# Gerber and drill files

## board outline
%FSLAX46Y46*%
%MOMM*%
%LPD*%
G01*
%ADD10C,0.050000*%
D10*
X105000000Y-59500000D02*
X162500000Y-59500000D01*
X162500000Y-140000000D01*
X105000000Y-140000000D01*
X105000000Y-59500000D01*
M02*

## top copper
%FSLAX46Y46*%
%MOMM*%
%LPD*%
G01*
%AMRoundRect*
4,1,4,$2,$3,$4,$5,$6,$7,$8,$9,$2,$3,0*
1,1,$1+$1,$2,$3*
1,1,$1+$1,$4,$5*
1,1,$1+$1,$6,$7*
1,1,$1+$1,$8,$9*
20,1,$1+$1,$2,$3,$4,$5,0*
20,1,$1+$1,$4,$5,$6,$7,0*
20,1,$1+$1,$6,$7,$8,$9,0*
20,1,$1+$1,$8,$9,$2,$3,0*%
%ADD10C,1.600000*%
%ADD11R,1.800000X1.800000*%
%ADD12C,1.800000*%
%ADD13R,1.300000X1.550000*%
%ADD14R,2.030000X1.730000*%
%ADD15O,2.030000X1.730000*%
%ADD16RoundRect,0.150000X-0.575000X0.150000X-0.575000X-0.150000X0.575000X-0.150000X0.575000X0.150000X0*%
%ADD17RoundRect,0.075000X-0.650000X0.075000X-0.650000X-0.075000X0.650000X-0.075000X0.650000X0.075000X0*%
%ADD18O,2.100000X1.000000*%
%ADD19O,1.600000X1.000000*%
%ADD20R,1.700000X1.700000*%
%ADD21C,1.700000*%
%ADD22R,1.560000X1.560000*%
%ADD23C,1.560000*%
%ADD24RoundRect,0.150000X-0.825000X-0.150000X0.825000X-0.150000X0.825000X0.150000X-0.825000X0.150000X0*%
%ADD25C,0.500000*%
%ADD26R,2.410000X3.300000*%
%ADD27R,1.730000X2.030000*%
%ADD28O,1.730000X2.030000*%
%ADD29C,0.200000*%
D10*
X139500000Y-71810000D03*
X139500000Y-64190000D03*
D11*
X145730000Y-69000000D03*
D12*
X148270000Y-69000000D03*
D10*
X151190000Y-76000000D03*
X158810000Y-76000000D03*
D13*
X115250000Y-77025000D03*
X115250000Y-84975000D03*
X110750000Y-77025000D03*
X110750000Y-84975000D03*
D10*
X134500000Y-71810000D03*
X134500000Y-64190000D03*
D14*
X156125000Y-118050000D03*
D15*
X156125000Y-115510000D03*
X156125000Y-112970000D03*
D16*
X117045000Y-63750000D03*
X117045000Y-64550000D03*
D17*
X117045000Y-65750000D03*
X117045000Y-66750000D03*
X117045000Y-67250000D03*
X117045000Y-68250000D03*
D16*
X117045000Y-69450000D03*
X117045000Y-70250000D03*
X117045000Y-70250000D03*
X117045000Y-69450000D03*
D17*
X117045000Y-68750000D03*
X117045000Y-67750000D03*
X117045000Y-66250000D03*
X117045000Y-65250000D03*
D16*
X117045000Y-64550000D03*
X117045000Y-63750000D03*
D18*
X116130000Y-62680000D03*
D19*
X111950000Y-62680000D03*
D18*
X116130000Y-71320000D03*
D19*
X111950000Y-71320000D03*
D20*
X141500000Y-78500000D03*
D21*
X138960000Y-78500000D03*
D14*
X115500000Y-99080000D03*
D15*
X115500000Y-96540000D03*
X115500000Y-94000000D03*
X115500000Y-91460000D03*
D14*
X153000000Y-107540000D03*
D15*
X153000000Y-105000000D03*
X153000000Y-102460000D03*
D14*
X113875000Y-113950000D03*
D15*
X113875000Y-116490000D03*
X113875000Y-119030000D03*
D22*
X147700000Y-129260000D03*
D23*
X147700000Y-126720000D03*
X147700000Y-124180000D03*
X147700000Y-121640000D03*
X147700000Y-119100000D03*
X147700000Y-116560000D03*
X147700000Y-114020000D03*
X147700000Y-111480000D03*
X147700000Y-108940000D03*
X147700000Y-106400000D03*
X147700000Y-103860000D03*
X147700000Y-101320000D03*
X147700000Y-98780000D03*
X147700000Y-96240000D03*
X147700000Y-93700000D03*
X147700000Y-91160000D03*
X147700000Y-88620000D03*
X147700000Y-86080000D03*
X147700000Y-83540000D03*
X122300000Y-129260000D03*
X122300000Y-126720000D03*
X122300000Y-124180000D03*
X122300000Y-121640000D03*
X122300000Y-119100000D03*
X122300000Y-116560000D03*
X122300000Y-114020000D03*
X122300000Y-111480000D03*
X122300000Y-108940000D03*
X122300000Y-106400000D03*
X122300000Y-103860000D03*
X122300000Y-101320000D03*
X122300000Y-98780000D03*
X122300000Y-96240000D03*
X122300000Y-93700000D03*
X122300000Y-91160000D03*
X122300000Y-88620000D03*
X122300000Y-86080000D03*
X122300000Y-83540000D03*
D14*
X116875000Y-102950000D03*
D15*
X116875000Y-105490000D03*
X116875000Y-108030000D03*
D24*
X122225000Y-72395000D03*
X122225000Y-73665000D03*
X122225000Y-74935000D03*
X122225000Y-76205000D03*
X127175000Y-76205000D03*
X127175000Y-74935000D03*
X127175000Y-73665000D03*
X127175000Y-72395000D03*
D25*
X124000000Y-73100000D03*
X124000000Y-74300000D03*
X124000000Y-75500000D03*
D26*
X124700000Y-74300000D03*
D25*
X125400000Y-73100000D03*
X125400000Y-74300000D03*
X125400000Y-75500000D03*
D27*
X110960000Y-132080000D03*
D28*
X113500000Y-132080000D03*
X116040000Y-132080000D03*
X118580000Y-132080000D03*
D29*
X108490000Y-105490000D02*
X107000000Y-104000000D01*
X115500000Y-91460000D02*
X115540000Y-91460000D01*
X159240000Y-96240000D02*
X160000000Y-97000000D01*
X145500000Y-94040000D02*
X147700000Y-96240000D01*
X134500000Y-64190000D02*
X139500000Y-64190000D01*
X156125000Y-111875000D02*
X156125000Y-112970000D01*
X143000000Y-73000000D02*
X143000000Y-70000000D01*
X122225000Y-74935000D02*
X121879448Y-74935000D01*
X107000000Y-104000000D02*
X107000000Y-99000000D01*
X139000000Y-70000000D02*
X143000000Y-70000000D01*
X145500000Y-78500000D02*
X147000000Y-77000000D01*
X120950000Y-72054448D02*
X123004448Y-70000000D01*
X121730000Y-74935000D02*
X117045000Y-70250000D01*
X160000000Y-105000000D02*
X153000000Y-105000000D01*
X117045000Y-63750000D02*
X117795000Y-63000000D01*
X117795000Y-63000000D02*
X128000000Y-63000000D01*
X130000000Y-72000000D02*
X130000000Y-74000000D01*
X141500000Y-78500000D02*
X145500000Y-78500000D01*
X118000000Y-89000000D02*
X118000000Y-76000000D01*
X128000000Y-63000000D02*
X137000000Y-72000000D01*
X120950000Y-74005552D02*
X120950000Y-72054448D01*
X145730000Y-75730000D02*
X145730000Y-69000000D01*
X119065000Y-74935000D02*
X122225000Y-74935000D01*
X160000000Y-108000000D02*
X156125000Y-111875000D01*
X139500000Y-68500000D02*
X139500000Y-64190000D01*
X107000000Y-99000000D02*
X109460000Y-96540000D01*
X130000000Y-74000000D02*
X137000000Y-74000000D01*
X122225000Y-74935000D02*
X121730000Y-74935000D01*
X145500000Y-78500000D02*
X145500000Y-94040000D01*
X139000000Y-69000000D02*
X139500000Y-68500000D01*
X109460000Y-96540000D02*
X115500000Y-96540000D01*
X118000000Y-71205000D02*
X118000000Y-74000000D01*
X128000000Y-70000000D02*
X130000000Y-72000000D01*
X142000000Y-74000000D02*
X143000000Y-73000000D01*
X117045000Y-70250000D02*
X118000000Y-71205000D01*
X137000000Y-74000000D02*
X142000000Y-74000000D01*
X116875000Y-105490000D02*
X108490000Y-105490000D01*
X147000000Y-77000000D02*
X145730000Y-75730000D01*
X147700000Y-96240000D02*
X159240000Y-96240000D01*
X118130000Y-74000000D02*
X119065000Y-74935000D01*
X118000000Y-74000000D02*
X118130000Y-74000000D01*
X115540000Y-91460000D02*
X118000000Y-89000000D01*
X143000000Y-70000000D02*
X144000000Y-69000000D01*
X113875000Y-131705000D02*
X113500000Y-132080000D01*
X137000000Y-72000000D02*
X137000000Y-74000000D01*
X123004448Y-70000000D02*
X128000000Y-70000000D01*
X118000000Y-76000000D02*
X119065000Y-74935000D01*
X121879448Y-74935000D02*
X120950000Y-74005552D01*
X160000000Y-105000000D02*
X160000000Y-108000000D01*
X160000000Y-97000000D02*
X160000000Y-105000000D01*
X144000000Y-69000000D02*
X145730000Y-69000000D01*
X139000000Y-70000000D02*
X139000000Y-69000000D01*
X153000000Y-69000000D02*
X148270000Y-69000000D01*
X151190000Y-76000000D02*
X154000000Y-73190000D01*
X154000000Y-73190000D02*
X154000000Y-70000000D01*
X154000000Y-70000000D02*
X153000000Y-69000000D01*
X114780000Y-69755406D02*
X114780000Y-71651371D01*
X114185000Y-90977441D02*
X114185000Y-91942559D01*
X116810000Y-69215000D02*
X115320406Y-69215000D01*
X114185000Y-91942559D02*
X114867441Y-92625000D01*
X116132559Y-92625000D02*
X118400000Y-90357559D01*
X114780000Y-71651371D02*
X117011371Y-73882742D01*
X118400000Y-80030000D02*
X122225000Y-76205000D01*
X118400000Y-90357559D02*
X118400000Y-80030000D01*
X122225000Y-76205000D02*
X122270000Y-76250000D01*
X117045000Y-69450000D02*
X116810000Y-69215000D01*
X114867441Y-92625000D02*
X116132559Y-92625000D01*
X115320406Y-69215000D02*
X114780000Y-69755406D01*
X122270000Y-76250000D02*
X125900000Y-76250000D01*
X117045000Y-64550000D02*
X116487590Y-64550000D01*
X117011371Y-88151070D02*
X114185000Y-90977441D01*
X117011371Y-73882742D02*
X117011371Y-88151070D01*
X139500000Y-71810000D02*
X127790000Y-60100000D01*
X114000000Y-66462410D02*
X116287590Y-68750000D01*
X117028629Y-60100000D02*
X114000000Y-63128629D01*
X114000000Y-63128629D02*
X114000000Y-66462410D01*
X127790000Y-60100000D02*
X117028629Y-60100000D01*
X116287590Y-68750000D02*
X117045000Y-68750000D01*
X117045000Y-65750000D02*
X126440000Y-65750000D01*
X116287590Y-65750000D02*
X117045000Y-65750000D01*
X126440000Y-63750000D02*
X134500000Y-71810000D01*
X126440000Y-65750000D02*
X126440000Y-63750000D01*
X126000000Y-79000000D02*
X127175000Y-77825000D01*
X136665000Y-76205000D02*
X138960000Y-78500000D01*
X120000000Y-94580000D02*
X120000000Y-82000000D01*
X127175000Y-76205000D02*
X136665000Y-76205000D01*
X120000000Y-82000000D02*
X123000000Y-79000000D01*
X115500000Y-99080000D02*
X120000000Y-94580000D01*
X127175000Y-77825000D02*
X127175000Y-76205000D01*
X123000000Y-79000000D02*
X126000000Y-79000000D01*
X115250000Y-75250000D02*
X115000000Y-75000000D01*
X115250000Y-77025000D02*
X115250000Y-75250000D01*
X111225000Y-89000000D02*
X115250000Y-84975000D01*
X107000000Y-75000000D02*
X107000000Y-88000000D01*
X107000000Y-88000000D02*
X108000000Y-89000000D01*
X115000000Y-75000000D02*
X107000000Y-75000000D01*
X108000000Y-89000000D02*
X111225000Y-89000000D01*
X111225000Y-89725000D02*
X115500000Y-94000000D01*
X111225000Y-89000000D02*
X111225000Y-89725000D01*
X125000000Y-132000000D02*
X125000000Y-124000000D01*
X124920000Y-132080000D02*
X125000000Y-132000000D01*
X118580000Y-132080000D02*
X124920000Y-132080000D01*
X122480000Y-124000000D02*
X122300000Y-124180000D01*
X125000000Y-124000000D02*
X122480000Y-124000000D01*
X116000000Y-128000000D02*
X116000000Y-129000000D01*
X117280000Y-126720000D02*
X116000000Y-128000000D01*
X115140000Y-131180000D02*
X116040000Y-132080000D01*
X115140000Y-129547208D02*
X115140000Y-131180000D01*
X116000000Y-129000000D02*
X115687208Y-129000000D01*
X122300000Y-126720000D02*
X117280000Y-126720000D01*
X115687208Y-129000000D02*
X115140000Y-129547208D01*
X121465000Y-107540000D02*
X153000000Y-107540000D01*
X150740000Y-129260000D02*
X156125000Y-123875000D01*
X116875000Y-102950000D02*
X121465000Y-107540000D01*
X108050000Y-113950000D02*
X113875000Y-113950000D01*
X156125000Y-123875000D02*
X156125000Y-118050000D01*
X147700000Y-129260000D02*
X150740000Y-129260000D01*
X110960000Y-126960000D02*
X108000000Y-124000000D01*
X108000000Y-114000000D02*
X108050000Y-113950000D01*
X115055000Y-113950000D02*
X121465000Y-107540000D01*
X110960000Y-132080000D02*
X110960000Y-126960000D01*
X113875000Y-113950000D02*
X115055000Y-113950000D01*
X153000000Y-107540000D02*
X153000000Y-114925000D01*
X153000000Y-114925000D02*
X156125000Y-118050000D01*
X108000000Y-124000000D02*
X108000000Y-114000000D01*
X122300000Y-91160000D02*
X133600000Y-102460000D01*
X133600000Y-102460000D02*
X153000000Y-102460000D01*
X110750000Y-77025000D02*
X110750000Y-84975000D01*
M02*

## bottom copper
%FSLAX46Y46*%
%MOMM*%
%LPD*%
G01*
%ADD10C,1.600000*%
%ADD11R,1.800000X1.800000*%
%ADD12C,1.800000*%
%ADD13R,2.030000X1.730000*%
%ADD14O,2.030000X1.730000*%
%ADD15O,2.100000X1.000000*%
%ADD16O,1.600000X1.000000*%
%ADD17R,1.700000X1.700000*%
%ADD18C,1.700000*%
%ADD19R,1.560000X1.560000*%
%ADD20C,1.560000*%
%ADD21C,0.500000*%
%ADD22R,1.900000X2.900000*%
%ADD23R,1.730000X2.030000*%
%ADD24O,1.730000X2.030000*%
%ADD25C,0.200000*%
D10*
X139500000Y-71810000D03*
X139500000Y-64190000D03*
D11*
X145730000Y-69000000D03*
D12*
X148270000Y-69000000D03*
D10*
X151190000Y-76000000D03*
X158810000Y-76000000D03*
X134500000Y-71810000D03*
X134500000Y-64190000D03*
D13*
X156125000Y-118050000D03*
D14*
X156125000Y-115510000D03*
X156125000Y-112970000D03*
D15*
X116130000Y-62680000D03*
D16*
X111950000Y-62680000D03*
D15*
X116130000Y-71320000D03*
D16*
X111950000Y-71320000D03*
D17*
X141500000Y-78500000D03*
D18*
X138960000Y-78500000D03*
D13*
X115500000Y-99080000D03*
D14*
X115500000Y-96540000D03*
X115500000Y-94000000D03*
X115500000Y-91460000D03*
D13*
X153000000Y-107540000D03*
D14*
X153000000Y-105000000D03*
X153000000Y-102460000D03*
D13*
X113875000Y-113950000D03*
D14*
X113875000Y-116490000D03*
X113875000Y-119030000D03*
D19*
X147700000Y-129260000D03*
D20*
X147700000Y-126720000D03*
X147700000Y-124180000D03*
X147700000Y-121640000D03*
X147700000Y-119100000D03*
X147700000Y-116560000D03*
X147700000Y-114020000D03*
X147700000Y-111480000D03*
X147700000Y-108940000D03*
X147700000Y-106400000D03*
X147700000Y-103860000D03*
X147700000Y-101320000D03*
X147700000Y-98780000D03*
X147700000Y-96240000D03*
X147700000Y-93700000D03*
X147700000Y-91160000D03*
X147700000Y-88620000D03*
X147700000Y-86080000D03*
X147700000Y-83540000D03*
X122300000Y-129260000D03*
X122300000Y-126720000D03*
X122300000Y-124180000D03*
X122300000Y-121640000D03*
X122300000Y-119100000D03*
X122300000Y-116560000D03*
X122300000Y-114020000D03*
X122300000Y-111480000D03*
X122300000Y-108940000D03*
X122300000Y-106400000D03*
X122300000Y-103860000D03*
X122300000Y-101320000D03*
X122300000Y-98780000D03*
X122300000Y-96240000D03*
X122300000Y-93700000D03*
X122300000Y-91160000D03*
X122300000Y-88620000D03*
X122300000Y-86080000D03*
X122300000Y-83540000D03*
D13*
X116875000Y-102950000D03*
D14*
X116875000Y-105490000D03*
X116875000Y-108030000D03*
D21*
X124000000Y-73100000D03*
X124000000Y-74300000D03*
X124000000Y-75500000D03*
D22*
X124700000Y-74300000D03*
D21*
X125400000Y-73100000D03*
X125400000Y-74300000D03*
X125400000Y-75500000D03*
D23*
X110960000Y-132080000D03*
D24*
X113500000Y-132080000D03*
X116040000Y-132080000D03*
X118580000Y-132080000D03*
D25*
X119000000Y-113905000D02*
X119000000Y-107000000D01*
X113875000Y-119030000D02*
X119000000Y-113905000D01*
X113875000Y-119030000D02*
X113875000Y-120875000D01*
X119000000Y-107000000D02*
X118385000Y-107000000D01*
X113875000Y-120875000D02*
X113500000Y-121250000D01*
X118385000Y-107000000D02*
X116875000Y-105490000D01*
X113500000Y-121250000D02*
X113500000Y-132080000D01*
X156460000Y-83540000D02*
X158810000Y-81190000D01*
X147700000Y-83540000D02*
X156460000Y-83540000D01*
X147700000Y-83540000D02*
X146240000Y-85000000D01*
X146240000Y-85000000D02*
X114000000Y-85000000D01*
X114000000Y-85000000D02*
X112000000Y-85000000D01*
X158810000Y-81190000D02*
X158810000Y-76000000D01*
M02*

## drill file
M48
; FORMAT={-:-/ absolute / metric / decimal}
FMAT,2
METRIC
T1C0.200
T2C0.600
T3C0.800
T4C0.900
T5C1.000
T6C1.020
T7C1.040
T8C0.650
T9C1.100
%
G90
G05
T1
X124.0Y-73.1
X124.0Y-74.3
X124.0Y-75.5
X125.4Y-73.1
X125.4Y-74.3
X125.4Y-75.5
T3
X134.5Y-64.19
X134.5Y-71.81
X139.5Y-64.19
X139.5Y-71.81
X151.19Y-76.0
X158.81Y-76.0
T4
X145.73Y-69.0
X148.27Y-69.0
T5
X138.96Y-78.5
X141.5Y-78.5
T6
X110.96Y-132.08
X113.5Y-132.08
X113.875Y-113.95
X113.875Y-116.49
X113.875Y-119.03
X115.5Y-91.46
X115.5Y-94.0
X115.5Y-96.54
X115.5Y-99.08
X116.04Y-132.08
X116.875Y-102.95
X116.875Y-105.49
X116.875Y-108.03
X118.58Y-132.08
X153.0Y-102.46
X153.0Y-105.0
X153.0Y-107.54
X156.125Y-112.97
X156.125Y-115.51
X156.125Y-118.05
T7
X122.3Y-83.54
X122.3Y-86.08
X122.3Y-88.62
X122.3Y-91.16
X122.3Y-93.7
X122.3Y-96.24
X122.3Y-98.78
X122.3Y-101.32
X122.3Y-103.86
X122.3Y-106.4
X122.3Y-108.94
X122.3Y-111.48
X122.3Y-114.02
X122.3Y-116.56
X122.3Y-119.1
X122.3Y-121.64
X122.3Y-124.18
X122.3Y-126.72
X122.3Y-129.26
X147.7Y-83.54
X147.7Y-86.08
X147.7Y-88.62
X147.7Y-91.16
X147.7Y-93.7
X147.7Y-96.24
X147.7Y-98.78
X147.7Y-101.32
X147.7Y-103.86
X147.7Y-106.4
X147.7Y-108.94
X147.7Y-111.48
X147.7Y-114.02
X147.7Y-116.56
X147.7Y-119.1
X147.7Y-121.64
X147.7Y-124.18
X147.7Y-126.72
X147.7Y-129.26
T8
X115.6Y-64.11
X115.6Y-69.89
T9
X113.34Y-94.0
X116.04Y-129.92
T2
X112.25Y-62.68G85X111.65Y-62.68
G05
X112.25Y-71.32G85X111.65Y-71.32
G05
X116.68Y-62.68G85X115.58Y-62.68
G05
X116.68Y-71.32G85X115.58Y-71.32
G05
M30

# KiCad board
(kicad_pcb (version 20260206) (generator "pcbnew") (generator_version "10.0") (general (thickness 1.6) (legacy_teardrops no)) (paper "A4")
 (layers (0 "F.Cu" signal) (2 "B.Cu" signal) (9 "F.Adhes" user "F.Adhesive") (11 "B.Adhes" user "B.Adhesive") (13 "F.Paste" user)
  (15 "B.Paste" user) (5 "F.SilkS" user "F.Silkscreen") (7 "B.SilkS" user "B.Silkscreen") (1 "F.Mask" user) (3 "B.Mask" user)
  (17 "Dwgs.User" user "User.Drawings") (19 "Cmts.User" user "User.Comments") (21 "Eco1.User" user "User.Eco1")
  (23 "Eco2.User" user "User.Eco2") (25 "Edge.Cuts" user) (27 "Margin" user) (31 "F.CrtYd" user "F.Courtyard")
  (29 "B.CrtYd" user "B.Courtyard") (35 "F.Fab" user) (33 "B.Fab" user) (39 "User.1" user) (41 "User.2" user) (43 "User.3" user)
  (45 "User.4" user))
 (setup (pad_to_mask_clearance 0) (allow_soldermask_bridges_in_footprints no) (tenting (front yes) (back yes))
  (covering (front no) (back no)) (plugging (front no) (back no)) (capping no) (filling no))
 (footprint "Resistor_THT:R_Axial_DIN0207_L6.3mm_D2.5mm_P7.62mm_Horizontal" (layer "F.Cu") (at 139.5 71.81 90)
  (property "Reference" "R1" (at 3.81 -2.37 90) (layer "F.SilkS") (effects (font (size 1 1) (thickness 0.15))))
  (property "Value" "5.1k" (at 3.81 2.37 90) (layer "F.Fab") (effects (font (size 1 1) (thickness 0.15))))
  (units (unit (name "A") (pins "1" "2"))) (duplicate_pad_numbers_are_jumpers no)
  (pad "1" thru_hole circle (at 0 0 90) (size 1.6 1.6) (drill 0.8) (layers "*.Cu" "*.Mask") (remove_unused_layers no) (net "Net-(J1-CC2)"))
  (pad "2" thru_hole circle (at 7.62 0 90) (size 1.6 1.6) (drill 0.8) (layers "*.Cu" "*.Mask") (remove_unused_layers no) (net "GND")))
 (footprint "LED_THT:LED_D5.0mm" (layer "F.Cu") (at 145.73 69)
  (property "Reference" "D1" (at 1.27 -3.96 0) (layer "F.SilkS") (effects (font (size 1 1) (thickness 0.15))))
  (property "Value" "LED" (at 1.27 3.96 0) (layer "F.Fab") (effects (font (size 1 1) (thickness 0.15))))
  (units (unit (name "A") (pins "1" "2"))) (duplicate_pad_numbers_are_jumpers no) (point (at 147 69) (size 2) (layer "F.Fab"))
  (pad "1" thru_hole rect (at 0 0) (size 1.8 1.8) (drill 0.9) (layers "*.Cu" "*.Mask") (remove_unused_layers no) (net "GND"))
  (pad "2" thru_hole circle (at 2.54 0) (size 1.8 1.8) (drill 0.9) (layers "*.Cu" "*.Mask") (remove_unused_layers no) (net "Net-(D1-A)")))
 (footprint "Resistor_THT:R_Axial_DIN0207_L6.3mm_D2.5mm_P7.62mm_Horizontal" (layer "F.Cu") (at 151.19 76)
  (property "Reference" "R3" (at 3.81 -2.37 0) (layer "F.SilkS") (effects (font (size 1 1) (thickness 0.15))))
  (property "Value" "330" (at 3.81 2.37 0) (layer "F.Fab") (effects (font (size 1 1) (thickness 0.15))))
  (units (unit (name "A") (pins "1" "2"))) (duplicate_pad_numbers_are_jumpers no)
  (pad "1" thru_hole circle (at 0 0) (size 1.6 1.6) (drill 0.8) (layers "*.Cu" "*.Mask") (remove_unused_layers no) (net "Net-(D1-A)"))
  (pad "2" thru_hole circle (at 7.62 0) (size 1.6 1.6) (drill 0.8) (layers "*.Cu" "*.Mask") (remove_unused_layers no) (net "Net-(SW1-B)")))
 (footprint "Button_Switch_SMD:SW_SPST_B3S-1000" (layer "F.Cu") (at 113 81 -90)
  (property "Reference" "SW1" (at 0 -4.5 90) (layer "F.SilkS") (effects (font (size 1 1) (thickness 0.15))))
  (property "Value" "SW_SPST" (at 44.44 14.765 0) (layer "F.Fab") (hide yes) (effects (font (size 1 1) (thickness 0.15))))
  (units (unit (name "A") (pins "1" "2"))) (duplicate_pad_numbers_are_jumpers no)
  (pad "1" smd rect (at -3.975 -2.25 270) (size 1.55 1.3) (layers "F.Cu" "F.Mask" "F.Paste") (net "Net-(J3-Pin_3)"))
  (pad "1" smd rect (at 3.975 -2.25 270) (size 1.55 1.3) (layers "F.Cu" "F.Mask" "F.Paste") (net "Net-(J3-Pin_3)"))
  (pad "2" smd rect (at -3.975 2.25 270) (size 1.55 1.3) (layers "F.Cu" "F.Mask" "F.Paste") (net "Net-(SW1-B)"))
  (pad "2" smd rect (at 3.975 2.25 270) (size 1.55 1.3) (layers "F.Cu" "F.Mask" "F.Paste") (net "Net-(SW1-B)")))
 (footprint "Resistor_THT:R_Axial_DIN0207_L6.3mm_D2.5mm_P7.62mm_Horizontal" (layer "F.Cu") (at 134.5 71.81 90)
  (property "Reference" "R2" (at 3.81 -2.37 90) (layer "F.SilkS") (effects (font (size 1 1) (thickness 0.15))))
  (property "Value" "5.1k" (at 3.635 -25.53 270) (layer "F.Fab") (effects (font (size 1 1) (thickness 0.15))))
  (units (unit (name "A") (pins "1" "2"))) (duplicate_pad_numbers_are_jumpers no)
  (pad "1" thru_hole circle (at 0 0 90) (size 1.6 1.6) (drill 0.8) (layers "*.Cu" "*.Mask") (remove_unused_layers no) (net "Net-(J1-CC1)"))
  (pad "2" thru_hole circle (at 7.62 0 90) (size 1.6 1.6) (drill 0.8) (layers "*.Cu" "*.Mask") (remove_unused_layers no) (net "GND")))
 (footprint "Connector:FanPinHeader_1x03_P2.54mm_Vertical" (layer "F.Cu") (at 156.125 118.05 90)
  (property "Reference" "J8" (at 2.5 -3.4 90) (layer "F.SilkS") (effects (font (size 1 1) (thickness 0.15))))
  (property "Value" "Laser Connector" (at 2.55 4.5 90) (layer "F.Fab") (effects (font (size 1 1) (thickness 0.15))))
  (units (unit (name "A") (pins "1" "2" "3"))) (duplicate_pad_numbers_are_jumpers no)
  (pad "1" thru_hole rect (at 0 0 180) (size 2.03 1.73) (drill 1.02) (layers "*.Cu" "*.Mask") (remove_unused_layers no)
   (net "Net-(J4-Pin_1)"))
  (pad "2" thru_hole oval (at 2.54 0 180) (size 2.03 1.73) (drill 1.02) (layers "*.Cu" "*.Mask") (remove_unused_layers no)
   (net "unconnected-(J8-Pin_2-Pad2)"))
  (pad "3" thru_hole oval (at 5.08 0 180) (size 2.03 1.73) (drill 1.02) (layers "*.Cu" "*.Mask") (remove_unused_layers no) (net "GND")))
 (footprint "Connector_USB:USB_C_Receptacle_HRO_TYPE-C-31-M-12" (layer "F.Cu") (at 113 67 -90)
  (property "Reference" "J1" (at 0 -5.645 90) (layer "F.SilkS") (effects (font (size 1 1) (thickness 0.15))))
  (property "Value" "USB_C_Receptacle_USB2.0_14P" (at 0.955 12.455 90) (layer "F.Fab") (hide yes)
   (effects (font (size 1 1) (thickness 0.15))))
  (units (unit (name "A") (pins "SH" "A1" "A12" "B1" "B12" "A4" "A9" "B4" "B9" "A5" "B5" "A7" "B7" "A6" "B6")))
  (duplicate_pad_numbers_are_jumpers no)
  (pad "" np_thru_hole circle (at -2.89 -2.6 270) (size 0.65 0.65) (drill 0.65) (layers "*.Cu" "*.Mask"))
  (pad "" np_thru_hole circle (at 2.89 -2.6 270) (size 0.65 0.65) (drill 0.65) (layers "*.Cu" "*.Mask"))
  (pad "A1" smd roundrect (at -3.25 -4.045 270) (size 0.6 1.45) (layers "F.Cu" "F.Mask" "F.Paste") (roundrect_rratio 0.25) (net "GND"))
  (pad "A4" smd roundrect (at -2.45 -4.045 270) (size 0.6 1.45) (layers "F.Cu" "F.Mask" "F.Paste") (roundrect_rratio 0.25)
   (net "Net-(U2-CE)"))
  (pad "A5" smd roundrect (at -1.25 -4.045 270) (size 0.3 1.45) (layers "F.Cu" "F.Mask" "F.Paste") (roundrect_rratio 0.25)
   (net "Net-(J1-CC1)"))
  (pad "A6" smd roundrect (at -0.25 -4.045 270) (size 0.3 1.45) (layers "F.Cu" "F.Mask" "F.Paste") (roundrect_rratio 0.25)
   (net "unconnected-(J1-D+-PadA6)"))
  (pad "A7" smd roundrect (at 0.25 -4.045 270) (size 0.3 1.45) (layers "F.Cu" "F.Mask" "F.Paste") (roundrect_rratio 0.25)
   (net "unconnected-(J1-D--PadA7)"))
  (pad "A8" smd roundrect (at 1.25 -4.045 270) (size 0.3 1.45) (layers "F.Cu" "F.Mask" "F.Paste") (roundrect_rratio 0.25))
  (pad "A9" smd roundrect (at 2.45 -4.045 270) (size 0.6 1.45) (layers "F.Cu" "F.Mask" "F.Paste") (roundrect_rratio 0.25)
   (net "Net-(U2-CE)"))
  (pad "A12" smd roundrect (at 3.25 -4.045 270) (size 0.6 1.45) (layers "F.Cu" "F.Mask" "F.Paste") (roundrect_rratio 0.25) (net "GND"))
  (pad "B1" smd roundrect (at 3.25 -4.045 270) (size 0.6 1.45) (layers "F.Cu" "F.Mask" "F.Paste") (roundrect_rratio 0.25) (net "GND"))
  (pad "B4" smd roundrect (at 2.45 -4.045 270) (size 0.6 1.45) (layers "F.Cu" "F.Mask" "F.Paste") (roundrect_rratio 0.25)
   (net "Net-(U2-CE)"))
  (pad "B5" smd roundrect (at 1.75 -4.045 270) (size 0.3 1.45) (layers "F.Cu" "F.Mask" "F.Paste") (roundrect_rratio 0.25)
   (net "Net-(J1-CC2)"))
  (pad "B6" smd roundrect (at 0.75 -4.045 270) (size 0.3 1.45) (layers "F.Cu" "F.Mask" "F.Paste") (roundrect_rratio 0.25)
   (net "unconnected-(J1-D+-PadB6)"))
  (pad "B7" smd roundrect (at -0.75 -4.045 270) (size 0.3 1.45) (layers "F.Cu" "F.Mask" "F.Paste") (roundrect_rratio 0.25)
   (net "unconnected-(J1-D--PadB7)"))
  (pad "B8" smd roundrect (at -1.75 -4.045 270) (size 0.3 1.45) (layers "F.Cu" "F.Mask" "F.Paste") (roundrect_rratio 0.25))
  (pad "B9" smd roundrect (at -2.45 -4.045 270) (size 0.6 1.45) (layers "F.Cu" "F.Mask" "F.Paste") (roundrect_rratio 0.25)
   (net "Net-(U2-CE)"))
  (pad "B12" smd roundrect (at -3.25 -4.045 270) (size 0.6 1.45) (layers "F.Cu" "F.Mask" "F.Paste") (roundrect_rratio 0.25) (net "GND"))
  (pad "SH" thru_hole oval (at -4.32 -3.13 270) (size 1 2.1) (drill oval 0.6 1.7) (layers "*.Cu" "*.Mask") (remove_unused_layers no)
   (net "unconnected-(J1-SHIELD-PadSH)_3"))
  (pad "SH" thru_hole oval (at -4.32 1.05 270) (size 1 1.6) (drill oval 0.6 1.2) (layers "*.Cu" "*.Mask") (remove_unused_layers no)
   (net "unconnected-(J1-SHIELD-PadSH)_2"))
  (pad "SH" thru_hole oval (at 4.32 -3.13 270) (size 1 2.1) (drill oval 0.6 1.7) (layers "*.Cu" "*.Mask") (remove_unused_layers no)
   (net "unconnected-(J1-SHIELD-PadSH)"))
  (pad "SH" thru_hole oval (at 4.32 1.05 270) (size 1 1.6) (drill oval 0.6 1.2) (layers "*.Cu" "*.Mask") (remove_unused_layers no)
   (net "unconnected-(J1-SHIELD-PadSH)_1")))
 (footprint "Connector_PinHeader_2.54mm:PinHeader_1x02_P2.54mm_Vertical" (layer "F.Cu") (at 141.5 78.5 -90)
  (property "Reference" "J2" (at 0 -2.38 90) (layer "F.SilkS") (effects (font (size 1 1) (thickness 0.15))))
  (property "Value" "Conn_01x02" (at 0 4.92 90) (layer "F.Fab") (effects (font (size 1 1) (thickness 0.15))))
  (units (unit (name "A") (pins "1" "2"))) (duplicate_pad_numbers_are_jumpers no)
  (pad "1" thru_hole rect (at 0 0 270) (size 1.7 1.7) (drill 1) (layers "*.Cu" "*.Mask") (remove_unused_layers no) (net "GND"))
  (pad "2" thru_hole circle (at 0 2.54 270) (size 1.7 1.7) (drill 1) (layers "*.Cu" "*.Mask") (remove_unused_layers no)
   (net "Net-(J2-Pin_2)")))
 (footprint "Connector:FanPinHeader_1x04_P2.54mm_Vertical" (layer "F.Cu") (at 115.5 99.08 90)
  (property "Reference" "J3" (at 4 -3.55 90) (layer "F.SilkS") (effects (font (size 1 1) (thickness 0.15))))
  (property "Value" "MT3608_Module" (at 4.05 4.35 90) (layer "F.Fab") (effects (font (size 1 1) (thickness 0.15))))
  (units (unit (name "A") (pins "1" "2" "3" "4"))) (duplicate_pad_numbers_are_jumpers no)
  (pad "" np_thru_hole circle (at 5.08 -2.16 180) (size 1.1 1.1) (drill 1.1) (layers "*.Cu" "*.Mask"))
  (pad "1" thru_hole rect (at 0 0 180) (size 2.03 1.73) (drill 1.02) (layers "*.Cu" "*.Mask") (remove_unused_layers no)
   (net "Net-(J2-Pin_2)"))
  (pad "2" thru_hole oval (at 2.54 0 180) (size 2.03 1.73) (drill 1.02) (layers "*.Cu" "*.Mask") (remove_unused_layers no) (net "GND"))
  (pad "3" thru_hole oval (at 5.08 0 180) (size 2.03 1.73) (drill 1.02) (layers "*.Cu" "*.Mask") (remove_unused_layers no)
   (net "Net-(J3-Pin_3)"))
  (pad "4" thru_hole oval (at 7.62 0 180) (size 2.03 1.73) (drill 1.02) (layers "*.Cu" "*.Mask") (remove_unused_layers no) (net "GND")))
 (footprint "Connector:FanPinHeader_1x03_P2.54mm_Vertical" (layer "F.Cu") (at 153 107.54 90)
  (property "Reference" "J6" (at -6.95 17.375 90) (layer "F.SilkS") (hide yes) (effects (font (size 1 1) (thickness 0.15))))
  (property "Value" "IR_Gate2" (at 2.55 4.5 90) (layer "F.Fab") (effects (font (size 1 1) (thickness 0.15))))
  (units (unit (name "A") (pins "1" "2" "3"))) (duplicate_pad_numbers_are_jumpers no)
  (pad "1" thru_hole rect (at 0 0 180) (size 2.03 1.73) (drill 1.02) (layers "*.Cu" "*.Mask") (remove_unused_layers no)
   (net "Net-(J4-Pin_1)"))
  (pad "2" thru_hole oval (at 2.54 0 180) (size 2.03 1.73) (drill 1.02) (layers "*.Cu" "*.Mask") (remove_unused_layers no) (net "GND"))
  (pad "3" thru_hole oval (at 5.08 0 180) (size 2.03 1.73) (drill 1.02) (layers "*.Cu" "*.Mask") (remove_unused_layers no)
   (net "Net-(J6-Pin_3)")))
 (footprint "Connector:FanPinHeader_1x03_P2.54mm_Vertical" (layer "F.Cu") (at 113.875 113.95 -90)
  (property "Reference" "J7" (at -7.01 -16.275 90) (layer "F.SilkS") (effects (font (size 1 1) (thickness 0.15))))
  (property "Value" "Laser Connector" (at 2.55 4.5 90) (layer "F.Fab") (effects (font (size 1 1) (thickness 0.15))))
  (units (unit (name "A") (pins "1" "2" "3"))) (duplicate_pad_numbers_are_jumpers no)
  (pad "1" thru_hole rect (at 0 0) (size 2.03 1.73) (drill 1.02) (layers "*.Cu" "*.Mask") (remove_unused_layers no) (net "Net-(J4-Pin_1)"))
  (pad "2" thru_hole oval (at 2.54 0) (size 2.03 1.73) (drill 1.02) (layers "*.Cu" "*.Mask") (remove_unused_layers no)
   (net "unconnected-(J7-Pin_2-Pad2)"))
  (pad "3" thru_hole oval (at 5.08 0) (size 2.03 1.73) (drill 1.02) (layers "*.Cu" "*.Mask") (remove_unused_layers no) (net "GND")))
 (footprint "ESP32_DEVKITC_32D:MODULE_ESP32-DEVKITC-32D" (layer "F.Cu") (at 135 109.5 180)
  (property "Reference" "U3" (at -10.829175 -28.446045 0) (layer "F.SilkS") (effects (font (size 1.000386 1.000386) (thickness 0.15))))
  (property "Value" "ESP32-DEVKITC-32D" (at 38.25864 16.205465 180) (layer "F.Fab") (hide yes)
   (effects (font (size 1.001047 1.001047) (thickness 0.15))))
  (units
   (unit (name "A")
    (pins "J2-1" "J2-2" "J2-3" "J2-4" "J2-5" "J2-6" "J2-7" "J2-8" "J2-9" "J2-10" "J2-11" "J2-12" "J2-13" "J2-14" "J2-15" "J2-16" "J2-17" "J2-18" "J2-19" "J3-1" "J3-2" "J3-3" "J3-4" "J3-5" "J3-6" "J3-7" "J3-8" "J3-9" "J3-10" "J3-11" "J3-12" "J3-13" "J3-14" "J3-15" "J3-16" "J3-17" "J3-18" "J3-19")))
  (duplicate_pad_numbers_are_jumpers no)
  (pad "J2-1" thru_hole rect (at -12.7 -19.76 180) (size 1.56 1.56) (drill 1.04) (layers "*.Cu" "*.Mask") (remove_unused_layers no)
   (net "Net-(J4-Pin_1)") (solder_mask_margin 0.102))
  (pad "J2-2" thru_hole circle (at -12.7 -17.22 180) (size 1.56 1.56) (drill 1.04) (layers "*.Cu" "*.Mask") (remove_unused_layers no)
   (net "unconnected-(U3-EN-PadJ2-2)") (solder_mask_margin 0.102))
  (pad "J2-3" thru_hole circle (at -12.7 -14.68 180) (size 1.56 1.56) (drill 1.04) (layers "*.Cu" "*.Mask") (remove_unused_layers no)
   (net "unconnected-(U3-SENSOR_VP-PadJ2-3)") (solder_mask_margin 0.102))
  (pad "J2-4" thru_hole circle (at -12.7 -12.14 180) (size 1.56 1.56) (drill 1.04) (layers "*.Cu" "*.Mask") (remove_unused_layers no)
   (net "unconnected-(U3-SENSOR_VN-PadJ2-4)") (solder_mask_margin 0.102))
  (pad "J2-5" thru_hole circle (at -12.7 -9.6 180) (size 1.56 1.56) (drill 1.04) (layers "*.Cu" "*.Mask") (remove_unused_layers no)
   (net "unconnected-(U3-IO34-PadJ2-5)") (solder_mask_margin 0.102))
  (pad "J2-6" thru_hole circle (at -12.7 -7.06 180) (size 1.56 1.56) (drill 1.04) (layers "*.Cu" "*.Mask") (remove_unused_layers no)
   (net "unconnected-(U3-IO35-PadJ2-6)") (solder_mask_margin 0.102))
  (pad "J2-7" thru_hole circle (at -12.7 -4.52 180) (size 1.56 1.56) (drill 1.04) (layers "*.Cu" "*.Mask") (remove_unused_layers no)
   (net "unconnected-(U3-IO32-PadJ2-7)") (solder_mask_margin 0.102))
  (pad "J2-8" thru_hole circle (at -12.7 -1.98 180) (size 1.56 1.56) (drill 1.04) (layers "*.Cu" "*.Mask") (remove_unused_layers no)
   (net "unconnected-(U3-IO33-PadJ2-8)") (solder_mask_margin 0.102))
  (pad "J2-9" thru_hole circle (at -12.7 0.56 180) (size 1.56 1.56) (drill 1.04) (layers "*.Cu" "*.Mask") (remove_unused_layers no)
   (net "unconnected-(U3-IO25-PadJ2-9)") (solder_mask_margin 0.102))
  (pad "J2-10" thru_hole circle (at -12.7 3.1 180) (size 1.56 1.56) (drill 1.04) (layers "*.Cu" "*.Mask") (remove_unused_layers no)
   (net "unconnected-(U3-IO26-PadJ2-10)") (solder_mask_margin 0.102))
  (pad "J2-11" thru_hole circle (at -12.7 5.64 180) (size 1.56 1.56) (drill 1.04) (layers "*.Cu" "*.Mask") (remove_unused_layers no)
   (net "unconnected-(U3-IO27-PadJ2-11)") (solder_mask_margin 0.102))
  (pad "J2-12" thru_hole circle (at -12.7 8.18 180) (size 1.56 1.56) (drill 1.04) (layers "*.Cu" "*.Mask") (remove_unused_layers no)
   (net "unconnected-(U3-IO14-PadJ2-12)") (solder_mask_margin 0.102))
  (pad "J2-13" thru_hole circle (at -12.7 10.72 180) (size 1.56 1.56) (drill 1.04) (layers "*.Cu" "*.Mask") (remove_unused_layers no)
   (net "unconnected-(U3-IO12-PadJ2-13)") (solder_mask_margin 0.102))
  (pad "J2-14" thru_hole circle (at -12.7 13.26 180) (size 1.56 1.56) (drill 1.04) (layers "*.Cu" "*.Mask") (remove_unused_layers no)
   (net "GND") (solder_mask_margin 0.102))
  (pad "J2-15" thru_hole circle (at -12.7 15.8 180) (size 1.56 1.56) (drill 1.04) (layers "*.Cu" "*.Mask") (remove_unused_layers no)
   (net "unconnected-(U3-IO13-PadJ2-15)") (solder_mask_margin 0.102))
  (pad "J2-16" thru_hole circle (at -12.7 18.34 180) (size 1.56 1.56) (drill 1.04) (layers "*.Cu" "*.Mask") (remove_unused_layers no)
   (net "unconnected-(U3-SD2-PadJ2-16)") (solder_mask_margin 0.102))
  (pad "J2-17" thru_hole circle (at -12.7 20.88 180) (size 1.56 1.56) (drill 1.04) (layers "*.Cu" "*.Mask") (remove_unused_layers no)
   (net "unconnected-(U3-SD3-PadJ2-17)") (solder_mask_margin 0.102))
  (pad "J2-18" thru_hole circle (at -12.7 23.42 180) (size 1.56 1.56) (drill 1.04) (layers "*.Cu" "*.Mask") (remove_unused_layers no)
   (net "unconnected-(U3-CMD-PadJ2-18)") (solder_mask_margin 0.102))
  (pad "J2-19" thru_hole circle (at -12.7 25.96 180) (size 1.56 1.56) (drill 1.04) (layers "*.Cu" "*.Mask") (remove_unused_layers no)
   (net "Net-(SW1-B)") (solder_mask_margin 0.102))
  (pad "J3-1" thru_hole circle (at 12.7 -19.76 180) (size 1.56 1.56) (drill 1.04) (layers "*.Cu" "*.Mask") (remove_unused_layers no)
   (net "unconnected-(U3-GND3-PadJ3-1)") (solder_mask_margin 0.102))
  (pad "J3-2" thru_hole circle (at 12.7 -17.22 180) (size 1.56 1.56) (drill 1.04) (layers "*.Cu" "*.Mask") (remove_unused_layers no)
   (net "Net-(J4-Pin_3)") (solder_mask_margin 0.102))
  (pad "J3-3" thru_hole circle (at 12.7 -14.68 180) (size 1.56 1.56) (drill 1.04) (layers "*.Cu" "*.Mask") (remove_unused_layers no)
   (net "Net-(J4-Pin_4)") (solder_mask_margin 0.102))
  (pad "J3-4" thru_hole circle (at 12.7 -12.14 180) (size 1.56 1.56) (drill 1.04) (layers "*.Cu" "*.Mask") (remove_unused_layers no)
   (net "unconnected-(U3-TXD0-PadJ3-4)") (solder_mask_margin 0.102))
  (pad "J3-5" thru_hole circle (at 12.7 -9.6 180) (size 1.56 1.56) (drill 1.04) (layers "*.Cu" "*.Mask") (remove_unused_layers no)
   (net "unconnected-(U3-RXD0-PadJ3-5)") (solder_mask_margin 0.102))
  (pad "J3-6" thru_hole circle (at 12.7 -7.06 180) (size 1.56 1.56) (drill 1.04) (layers "*.Cu" "*.Mask") (remove_unused_layers no)
   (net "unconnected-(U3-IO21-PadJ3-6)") (solder_mask_margin 0.102))
  (pad "J3-7" thru_hole circle (at 12.7 -4.52 180) (size 1.56 1.56) (drill 1.04) (layers "*.Cu" "*.Mask") (remove_unused_layers no)
   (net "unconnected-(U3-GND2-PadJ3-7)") (solder_mask_margin 0.102))
  (pad "J3-8" thru_hole circle (at 12.7 -1.98 180) (size 1.56 1.56) (drill 1.04) (layers "*.Cu" "*.Mask") (remove_unused_layers no)
   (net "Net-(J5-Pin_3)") (solder_mask_margin 0.102))
  (pad "J3-9" thru_hole circle (at 12.7 0.56 180) (size 1.56 1.56) (drill 1.04) (layers "*.Cu" "*.Mask") (remove_unused_layers no)
   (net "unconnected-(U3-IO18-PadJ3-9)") (solder_mask_margin 0.102))
  (pad "J3-10" thru_hole circle (at 12.7 3.1 180) (size 1.56 1.56) (drill 1.04) (layers "*.Cu" "*.Mask") (remove_unused_layers no)
   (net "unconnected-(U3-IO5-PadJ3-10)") (solder_mask_margin 0.102))
  (pad "J3-11" thru_hole circle (at 12.7 5.64 180) (size 1.56 1.56) (drill 1.04) (layers "*.Cu" "*.Mask") (remove_unused_layers no)
   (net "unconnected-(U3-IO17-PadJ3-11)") (solder_mask_margin 0.102))
  (pad "J3-12" thru_hole circle (at 12.7 8.18 180) (size 1.56 1.56) (drill 1.04) (layers "*.Cu" "*.Mask") (remove_unused_layers no)
   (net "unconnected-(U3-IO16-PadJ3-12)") (solder_mask_margin 0.102))
  (pad "J3-13" thru_hole circle (at 12.7 10.72 180) (size 1.56 1.56) (drill 1.04) (layers "*.Cu" "*.Mask") (remove_unused_layers no)
   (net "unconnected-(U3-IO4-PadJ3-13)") (solder_mask_margin 0.102))
  (pad "J3-14" thru_hole circle (at 12.7 13.26 180) (size 1.56 1.56) (drill 1.04) (layers "*.Cu" "*.Mask") (remove_unused_layers no)
   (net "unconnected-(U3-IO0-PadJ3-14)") (solder_mask_margin 0.102))
  (pad "J3-15" thru_hole circle (at 12.7 15.8 180) (size 1.56 1.56) (drill 1.04) (layers "*.Cu" "*.Mask") (remove_unused_layers no)
   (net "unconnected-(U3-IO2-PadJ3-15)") (solder_mask_margin 0.102))
  (pad "J3-16" thru_hole circle (at 12.7 18.34 180) (size 1.56 1.56) (drill 1.04) (layers "*.Cu" "*.Mask") (remove_unused_layers no)
   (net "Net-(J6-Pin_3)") (solder_mask_margin 0.102))
  (pad "J3-17" thru_hole circle (at 12.7 20.88 180) (size 1.56 1.56) (drill 1.04) (layers "*.Cu" "*.Mask") (remove_unused_layers no)
   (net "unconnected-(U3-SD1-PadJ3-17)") (solder_mask_margin 0.102))
  (pad "J3-18" thru_hole circle (at 12.7 23.42 180) (size 1.56 1.56) (drill 1.04) (layers "*.Cu" "*.Mask") (remove_unused_layers no)
   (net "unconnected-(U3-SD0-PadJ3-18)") (solder_mask_margin 0.102))
  (pad "J3-19" thru_hole circle (at 12.7 25.96 180) (size 1.56 1.56) (drill 1.04) (layers "*.Cu" "*.Mask") (remove_unused_layers no)
   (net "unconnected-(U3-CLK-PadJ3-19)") (solder_mask_margin 0.102)))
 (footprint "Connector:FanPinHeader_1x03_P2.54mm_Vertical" (layer "F.Cu") (at 116.875 102.95 -90)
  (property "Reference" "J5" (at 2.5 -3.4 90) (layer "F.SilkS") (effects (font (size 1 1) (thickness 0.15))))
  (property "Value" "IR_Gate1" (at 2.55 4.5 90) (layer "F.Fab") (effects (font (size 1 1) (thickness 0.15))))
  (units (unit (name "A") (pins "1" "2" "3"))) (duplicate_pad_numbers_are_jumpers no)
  (pad "1" thru_hole rect (at 0 0) (size 2.03 1.73) (drill 1.02) (layers "*.Cu" "*.Mask") (remove_unused_layers no) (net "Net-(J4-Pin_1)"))
  (pad "2" thru_hole oval (at 2.54 0) (size 2.03 1.73) (drill 1.02) (layers "*.Cu" "*.Mask") (remove_unused_layers no) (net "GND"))
  (pad "3" thru_hole oval (at 5.08 0) (size 2.03 1.73) (drill 1.02) (layers "*.Cu" "*.Mask") (remove_unused_layers no)
   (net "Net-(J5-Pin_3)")))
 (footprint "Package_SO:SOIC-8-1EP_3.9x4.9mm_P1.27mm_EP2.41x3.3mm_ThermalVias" (layer "F.Cu") (at 124.7 74.3)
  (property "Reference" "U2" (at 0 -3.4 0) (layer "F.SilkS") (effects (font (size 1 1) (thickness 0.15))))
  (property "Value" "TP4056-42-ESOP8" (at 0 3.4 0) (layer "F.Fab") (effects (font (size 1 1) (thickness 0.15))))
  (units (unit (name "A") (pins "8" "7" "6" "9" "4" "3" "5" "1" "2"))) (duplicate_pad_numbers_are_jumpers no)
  (pad "" smd roundrect (at -0.6 -0.825) (size 1.01 1.38) (layers "F.Paste") (roundrect_rratio 0.247525))
  (pad "" smd roundrect (at -0.6 0.825) (size 1.01 1.38) (layers "F.Paste") (roundrect_rratio 0.247525))
  (pad "" smd roundrect (at 0.6 -0.825) (size 1.01 1.38) (layers "F.Paste") (roundrect_rratio 0.247525))
  (pad "" smd roundrect (at 0.6 0.825) (size 1.01 1.38) (layers "F.Paste") (roundrect_rratio 0.247525))
  (pad "1" smd roundrect (at -2.475 -1.905) (size 1.95 0.6) (layers "F.Cu" "F.Mask" "F.Paste") (roundrect_rratio 0.25)
   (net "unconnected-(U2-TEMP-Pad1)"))
  (pad "2" smd roundrect (at -2.475 -0.635) (size 1.95 0.6) (layers "F.Cu" "F.Mask" "F.Paste") (roundrect_rratio 0.25)
   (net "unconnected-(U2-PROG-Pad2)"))
  (pad "3" smd roundrect (at -2.475 0.635) (size 1.95 0.6) (layers "F.Cu" "F.Mask" "F.Paste") (roundrect_rratio 0.25) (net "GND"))
  (pad "4" smd roundrect (at -2.475 1.905) (size 1.95 0.6) (layers "F.Cu" "F.Mask" "F.Paste") (roundrect_rratio 0.25) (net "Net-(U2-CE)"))
  (pad "5" smd roundrect (at 2.475 1.905) (size 1.95 0.6) (layers "F.Cu" "F.Mask" "F.Paste") (roundrect_rratio 0.25) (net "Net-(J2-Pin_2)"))
  (pad "6" smd roundrect (at 2.475 0.635) (size 1.95 0.6) (layers "F.Cu" "F.Mask" "F.Paste") (roundrect_rratio 0.25)
   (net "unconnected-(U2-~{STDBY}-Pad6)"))
  (pad "7" smd roundrect (at 2.475 -0.635) (size 1.95 0.6) (layers "F.Cu" "F.Mask" "F.Paste") (roundrect_rratio 0.25)
   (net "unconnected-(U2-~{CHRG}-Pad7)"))
  (pad "8" smd roundrect (at 2.475 -1.905) (size 1.95 0.6) (layers "F.Cu" "F.Mask" "F.Paste") (roundrect_rratio 0.25) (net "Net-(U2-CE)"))
  (pad "9" thru_hole circle (at -0.7 -1.2) (size 0.5 0.5) (drill 0.2) (layers "*.Cu") (remove_unused_layers no)
   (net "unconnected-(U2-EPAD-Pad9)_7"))
  (pad "9" thru_hole circle (at -0.7 0) (size 0.5 0.5) (drill 0.2) (layers "*.Cu") (remove_unused_layers no)
   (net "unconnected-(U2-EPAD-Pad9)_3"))
  (pad "9" thru_hole circle (at -0.7 1.2) (size 0.5 0.5) (drill 0.2) (layers "*.Cu") (remove_unused_layers no)
   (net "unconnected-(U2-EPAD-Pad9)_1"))
  (pad "9" smd rect (at 0 0) (size 1.9 2.9) (layers "B.Cu") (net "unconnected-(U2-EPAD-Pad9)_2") (zone_connect 2))
  (pad "9" smd rect (at 0 0) (size 2.41 3.3) (layers "F.Cu" "F.Mask") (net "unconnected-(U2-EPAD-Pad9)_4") (zone_connect 2))
  (pad "9" thru_hole circle (at 0.7 -1.2) (size 0.5 0.5) (drill 0.2) (layers "*.Cu") (remove_unused_layers no)
   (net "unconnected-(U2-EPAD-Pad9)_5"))
  (pad "9" thru_hole circle (at 0.7 0) (size 0.5 0.5) (drill 0.2) (layers "*.Cu") (remove_unused_layers no)
   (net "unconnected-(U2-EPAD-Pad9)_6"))
  (pad "9" thru_hole circle (at 0.7 1.2) (size 0.5 0.5) (drill 0.2) (layers "*.Cu") (remove_unused_layers no)
   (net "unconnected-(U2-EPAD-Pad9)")))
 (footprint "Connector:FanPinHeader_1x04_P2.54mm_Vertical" (layer "F.Cu") (at 110.96 132.08)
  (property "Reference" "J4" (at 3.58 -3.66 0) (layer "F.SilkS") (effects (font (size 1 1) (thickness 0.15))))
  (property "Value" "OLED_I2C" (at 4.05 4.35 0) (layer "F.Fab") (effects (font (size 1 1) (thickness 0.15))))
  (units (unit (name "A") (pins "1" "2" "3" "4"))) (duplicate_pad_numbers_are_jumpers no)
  (pad "" np_thru_hole circle (at 5.08 -2.16 90) (size 1.1 1.1) (drill 1.1) (layers "*.Cu" "*.Mask"))
  (pad "1" thru_hole rect (at 0 0 90) (size 2.03 1.73) (drill 1.02) (layers "*.Cu" "*.Mask") (remove_unused_layers no)
   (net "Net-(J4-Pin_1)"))
  (pad "2" thru_hole oval (at 2.54 0 90) (size 2.03 1.73) (drill 1.02) (layers "*.Cu" "*.Mask") (remove_unused_layers no) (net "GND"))
  (pad "3" thru_hole oval (at 5.08 0 90) (size 2.03 1.73) (drill 1.02) (layers "*.Cu" "*.Mask") (remove_unused_layers no)
   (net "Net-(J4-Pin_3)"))
  (pad "4" thru_hole oval (at 7.62 0 90) (size 2.03 1.73) (drill 1.02) (layers "*.Cu" "*.Mask") (remove_unused_layers no)
   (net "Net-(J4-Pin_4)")))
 (gr_rect (start 105 59.5) (end 162.5 140) (stroke (width 0.05) (type default)) (fill no) (layer "Edge.Cuts"))
 (segment (start 108.49 105.49) (end 107 104) (width 0.2) (layer "F.Cu") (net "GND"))
 (segment (start 115.5 91.46) (end 115.54 91.46) (width 0.2) (layer "F.Cu") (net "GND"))
 (segment (start 159.24 96.24) (end 160 97) (width 0.2) (layer "F.Cu") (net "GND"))
 (segment (start 145.5 94.04) (end 147.7 96.24) (width 0.2) (layer "F.Cu") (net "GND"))
 (segment (start 134.5 64.19) (end 139.5 64.19) (width 0.2) (layer "F.Cu") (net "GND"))
 (segment (start 156.125 111.875) (end 156.125 112.97) (width 0.2) (layer "F.Cu") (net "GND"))
 (segment (start 143 73) (end 143 70) (width 0.2) (layer "F.Cu") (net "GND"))
 (segment (start 122.225 74.935) (end 121.879448 74.935) (width 0.2) (layer "F.Cu") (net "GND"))
 (segment (start 107 104) (end 107 99) (width 0.2) (layer "F.Cu") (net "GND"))
 (segment (start 139 70) (end 143 70) (width 0.2) (layer "F.Cu") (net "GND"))
 (segment (start 145.5 78.5) (end 147 77) (width 0.2) (layer "F.Cu") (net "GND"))
 (segment (start 120.95 72.054448) (end 123.004448 70) (width 0.2) (layer "F.Cu") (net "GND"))
 (segment (start 121.73 74.935) (end 117.045 70.25) (width 0.2) (layer "F.Cu") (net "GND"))
 (segment (start 160 105) (end 153 105) (width 0.2) (layer "F.Cu") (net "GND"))
 (segment (start 117.045 63.75) (end 117.795 63) (width 0.2) (layer "F.Cu") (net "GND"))
 (segment (start 117.795 63) (end 128 63) (width 0.2) (layer "F.Cu") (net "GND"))
 (segment (start 130 72) (end 130 74) (width 0.2) (layer "F.Cu") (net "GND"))
 (segment (start 141.5 78.5) (end 145.5 78.5) (width 0.2) (layer "F.Cu") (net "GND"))
 (segment (start 118 89) (end 118 76) (width 0.2) (layer "F.Cu") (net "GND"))
 (segment (start 128 63) (end 137 72) (width 0.2) (layer "F.Cu") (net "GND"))
 (segment (start 120.95 74.005552) (end 120.95 72.054448) (width 0.2) (layer "F.Cu") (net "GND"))
 (segment (start 145.73 75.73) (end 145.73 69) (width 0.2) (layer "F.Cu") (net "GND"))
 (segment (start 119.065 74.935) (end 122.225 74.935) (width 0.2) (layer "F.Cu") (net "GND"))
 (segment (start 160 108) (end 156.125 111.875) (width 0.2) (layer "F.Cu") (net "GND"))
 (segment (start 139.5 68.5) (end 139.5 64.19) (width 0.2) (layer "F.Cu") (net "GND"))
 (segment (start 107 99) (end 109.46 96.54) (width 0.2) (layer "F.Cu") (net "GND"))
 (segment (start 130 74) (end 137 74) (width 0.2) (layer "F.Cu") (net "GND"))
 (segment (start 122.225 74.935) (end 121.73 74.935) (width 0.2) (layer "F.Cu") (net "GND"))
 (segment (start 145.5 78.5) (end 145.5 94.04) (width 0.2) (layer "F.Cu") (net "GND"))
 (segment (start 139 69) (end 139.5 68.5) (width 0.2) (layer "F.Cu") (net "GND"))
 (segment (start 109.46 96.54) (end 115.5 96.54) (width 0.2) (layer "F.Cu") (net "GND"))
 (segment (start 118 71.205) (end 118 74) (width 0.2) (layer "F.Cu") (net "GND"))
 (segment (start 128 70) (end 130 72) (width 0.2) (layer "F.Cu") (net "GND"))
 (segment (start 142 74) (end 143 73) (width 0.2) (layer "F.Cu") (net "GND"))
 (segment (start 117.045 70.25) (end 118 71.205) (width 0.2) (layer "F.Cu") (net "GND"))
 (segment (start 137 74) (end 142 74) (width 0.2) (layer "F.Cu") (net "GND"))
 (segment (start 116.875 105.49) (end 108.49 105.49) (width 0.2) (layer "F.Cu") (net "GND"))
 (segment (start 147 77) (end 145.73 75.73) (width 0.2) (layer "F.Cu") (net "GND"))
 (segment (start 147.7 96.24) (end 159.24 96.24) (width 0.2) (layer "F.Cu") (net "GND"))
 (segment (start 118.13 74) (end 119.065 74.935) (width 0.2) (layer "F.Cu") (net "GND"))
 (segment (start 118 74) (end 118.13 74) (width 0.2) (layer "F.Cu") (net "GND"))
 (segment (start 115.54 91.46) (end 118 89) (width 0.2) (layer "F.Cu") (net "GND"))
 (segment (start 143 70) (end 144 69) (width 0.2) (layer "F.Cu") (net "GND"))
 (segment (start 113.875 131.705) (end 113.5 132.08) (width 0.2) (layer "F.Cu") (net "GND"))
 (segment (start 137 72) (end 137 74) (width 0.2) (layer "F.Cu") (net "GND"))
 (segment (start 123.004448 70) (end 128 70) (width 0.2) (layer "F.Cu") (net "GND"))
 (segment (start 118 76) (end 119.065 74.935) (width 0.2) (layer "F.Cu") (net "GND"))
 (segment (start 121.879448 74.935) (end 120.95 74.005552) (width 0.2) (layer "F.Cu") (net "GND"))
 (segment (start 160 105) (end 160 108) (width 0.2) (layer "F.Cu") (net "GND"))
 (segment (start 160 97) (end 160 105) (width 0.2) (layer "F.Cu") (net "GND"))
 (segment (start 144 69) (end 145.73 69) (width 0.2) (layer "F.Cu") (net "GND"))
 (segment (start 139 70) (end 139 69) (width 0.2) (layer "F.Cu") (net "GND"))
 (segment (start 119 113.905) (end 119 107) (width 0.2) (layer "B.Cu") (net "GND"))
 (segment (start 113.875 119.03) (end 119 113.905) (width 0.2) (layer "B.Cu") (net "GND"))
 (segment (start 113.875 119.03) (end 113.875 120.875) (width 0.2) (layer "B.Cu") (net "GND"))
 (segment (start 119 107) (end 118.385 107) (width 0.2) (layer "B.Cu") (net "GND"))
 (segment (start 113.875 120.875) (end 113.5 121.25) (width 0.2) (layer "B.Cu") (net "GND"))
 (segment (start 118.385 107) (end 116.875 105.49) (width 0.2) (layer "B.Cu") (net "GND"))
 (segment (start 113.5 121.25) (end 113.5 132.08) (width 0.2) (layer "B.Cu") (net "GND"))
 (segment (start 153 69) (end 148.27 69) (width 0.2) (layer "F.Cu") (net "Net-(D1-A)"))
 (segment (start 151.19 76) (end 154 73.19) (width 0.2) (layer "F.Cu") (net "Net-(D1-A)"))
 (segment (start 154 73.19) (end 154 70) (width 0.2) (layer "F.Cu") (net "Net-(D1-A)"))
 (segment (start 154 70) (end 153 69) (width 0.2) (layer "F.Cu") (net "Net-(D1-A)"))
 (segment (start 114.78 69.755406) (end 114.78 71.651371) (width 0.2) (layer "F.Cu") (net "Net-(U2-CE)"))
 (segment (start 114.185 90.977441) (end 114.185 91.942559) (width 0.2) (layer "F.Cu") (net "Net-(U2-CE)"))
 (segment (start 116.81 69.215) (end 115.320406 69.215) (width 0.2) (layer "F.Cu") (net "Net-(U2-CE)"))
 (segment (start 114.185 91.942559) (end 114.867441 92.625) (width 0.2) (layer "F.Cu") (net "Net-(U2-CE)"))
 (segment (start 116.132559 92.625) (end 118.4 90.357559) (width 0.2) (layer "F.Cu") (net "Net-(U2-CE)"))
 (segment (start 114.78 71.651371) (end 117.011371 73.882742) (width 0.2) (layer "F.Cu") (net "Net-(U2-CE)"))
 (segment (start 118.4 80.03) (end 122.225 76.205) (width 0.2) (layer "F.Cu") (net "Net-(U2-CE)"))
 (segment (start 118.4 90.357559) (end 118.4 80.03) (width 0.2) (layer "F.Cu") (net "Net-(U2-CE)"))
 (segment (start 122.225 76.205) (end 122.27 76.25) (width 0.2) (layer "F.Cu") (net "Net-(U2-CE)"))
 (segment (start 117.045 69.45) (end 116.81 69.215) (width 0.2) (layer "F.Cu") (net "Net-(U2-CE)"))
 (segment (start 114.867441 92.625) (end 116.132559 92.625) (width 0.2) (layer "F.Cu") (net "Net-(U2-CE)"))
 (segment (start 115.320406 69.215) (end 114.78 69.755406) (width 0.2) (layer "F.Cu") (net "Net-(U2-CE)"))
 (segment (start 122.27 76.25) (end 125.9 76.25) (width 0.2) (layer "F.Cu") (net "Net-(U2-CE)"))
 (segment (start 117.045 64.55) (end 116.48759 64.55) (width 0.2) (layer "F.Cu") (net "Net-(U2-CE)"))
 (segment (start 117.011371 88.15107) (end 114.185 90.977441) (width 0.2) (layer "F.Cu") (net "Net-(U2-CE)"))
 (segment (start 117.011371 73.882742) (end 117.011371 88.15107) (width 0.2) (layer "F.Cu") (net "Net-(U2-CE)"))
 (segment (start 139.5 71.81) (end 127.79 60.1) (width 0.2) (layer "F.Cu") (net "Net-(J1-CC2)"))
 (segment (start 114 66.46241) (end 116.28759 68.75) (width 0.2) (layer "F.Cu") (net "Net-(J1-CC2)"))
 (segment (start 117.028629 60.1) (end 114 63.128629) (width 0.2) (layer "F.Cu") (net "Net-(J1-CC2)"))
 (segment (start 114 63.128629) (end 114 66.46241) (width 0.2) (layer "F.Cu") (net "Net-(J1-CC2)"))
 (segment (start 127.79 60.1) (end 117.028629 60.1) (width 0.2) (layer "F.Cu") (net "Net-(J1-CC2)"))
 (segment (start 116.28759 68.75) (end 117.045 68.75) (width 0.2) (layer "F.Cu") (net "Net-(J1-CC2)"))
 (segment (start 117.045 65.75) (end 126.44 65.75) (width 0.2) (layer "F.Cu") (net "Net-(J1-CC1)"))
 (segment (start 116.28759 65.75) (end 117.045 65.75) (width 0.2) (layer "F.Cu") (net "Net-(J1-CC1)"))
 (segment (start 126.44 63.75) (end 134.5 71.81) (width 0.2) (layer "F.Cu") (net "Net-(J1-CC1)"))
 (segment (start 126.44 65.75) (end 126.44 63.75) (width 0.2) (layer "F.Cu") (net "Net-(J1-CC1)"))
 (segment (start 126 79) (end 127.175 77.825) (width 0.2) (layer "F.Cu") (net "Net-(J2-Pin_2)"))
 (segment (start 136.665 76.205) (end 138.96 78.5) (width 0.2) (layer "F.Cu") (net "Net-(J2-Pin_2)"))
 (segment (start 120 94.58) (end 120 82) (width 0.2) (layer "F.Cu") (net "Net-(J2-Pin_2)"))
 (segment (start 127.175 76.205) (end 136.665 76.205) (width 0.2) (layer "F.Cu") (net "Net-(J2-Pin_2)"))
 (segment (start 120 82) (end 123 79) (width 0.2) (layer "F.Cu") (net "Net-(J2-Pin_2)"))
 (segment (start 115.5 99.08) (end 120 94.58) (width 0.2) (layer "F.Cu") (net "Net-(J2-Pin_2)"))
 (segment (start 127.175 77.825) (end 127.175 76.205) (width 0.2) (layer "F.Cu") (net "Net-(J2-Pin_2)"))
 (segment (start 123 79) (end 126 79) (width 0.2) (layer "F.Cu") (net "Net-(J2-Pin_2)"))
 (segment (start 115.25 75.25) (end 115 75) (width 0.2) (layer "F.Cu") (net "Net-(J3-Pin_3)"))
 (segment (start 115.25 77.025) (end 115.25 75.25) (width 0.2) (layer "F.Cu") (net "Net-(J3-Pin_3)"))
 (segment (start 111.225 89) (end 115.25 84.975) (width 0.2) (layer "F.Cu") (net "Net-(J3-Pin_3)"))
 (segment (start 107 75) (end 107 88) (width 0.2) (layer "F.Cu") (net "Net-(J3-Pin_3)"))
 (segment (start 107 88) (end 108 89) (width 0.2) (layer "F.Cu") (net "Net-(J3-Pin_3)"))
 (segment (start 115 75) (end 107 75) (width 0.2) (layer "F.Cu") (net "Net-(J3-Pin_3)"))
 (segment (start 108 89) (end 111.225 89) (width 0.2) (layer "F.Cu") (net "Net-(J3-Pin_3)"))
 (segment (start 111.225 89.725) (end 115.5 94) (width 0.2) (layer "F.Cu") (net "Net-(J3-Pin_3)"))
 (segment (start 111.225 89) (end 111.225 89.725) (width 0.2) (layer "F.Cu") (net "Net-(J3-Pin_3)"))
 (segment (start 125 132) (end 125 124) (width 0.2) (layer "F.Cu") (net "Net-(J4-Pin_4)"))
 (segment (start 124.92 132.08) (end 125 132) (width 0.2) (layer "F.Cu") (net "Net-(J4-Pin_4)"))
 (segment (start 118.58 132.08) (end 124.92 132.08) (width 0.2) (layer "F.Cu") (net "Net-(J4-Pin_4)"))
 (segment (start 122.48 124) (end 122.3 124.18) (width 0.2) (layer "F.Cu") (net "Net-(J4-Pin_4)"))
 (segment (start 125 124) (end 122.48 124) (width 0.2) (layer "F.Cu") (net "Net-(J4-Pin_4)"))
 (segment (start 116 128) (end 116 129) (width 0.2) (layer "F.Cu") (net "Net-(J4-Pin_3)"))
 (segment (start 117.28 126.72) (end 116 128) (width 0.2) (layer "F.Cu") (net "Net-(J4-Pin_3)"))
 (segment (start 115.14 131.18) (end 116.04 132.08) (width 0.2) (layer "F.Cu") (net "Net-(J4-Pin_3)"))
 (segment (start 115.14 129.547208) (end 115.14 131.18) (width 0.2) (layer "F.Cu") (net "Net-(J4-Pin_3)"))
 (segment (start 116 129) (end 115.687208 129) (width 0.2) (layer "F.Cu") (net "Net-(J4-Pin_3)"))
 (segment (start 122.3 126.72) (end 117.28 126.72) (width 0.2) (layer "F.Cu") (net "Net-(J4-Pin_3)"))
 (segment (start 115.687208 129) (end 115.14 129.547208) (width 0.2) (layer "F.Cu") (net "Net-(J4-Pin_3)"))
 (segment (start 121.465 107.54) (end 153 107.54) (width 0.2) (layer "F.Cu") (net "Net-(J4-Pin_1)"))
 (segment (start 150.74 129.26) (end 156.125 123.875) (width 0.2) (layer "F.Cu") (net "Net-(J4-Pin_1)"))
 (segment (start 116.875 102.95) (end 121.465 107.54) (width 0.2) (layer "F.Cu") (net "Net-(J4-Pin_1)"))
 (segment (start 108.05 113.95) (end 113.875 113.95) (width 0.2) (layer "F.Cu") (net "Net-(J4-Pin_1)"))
 (segment (start 156.125 123.875) (end 156.125 118.05) (width 0.2) (layer "F.Cu") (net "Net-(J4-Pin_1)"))
 (segment (start 147.7 129.26) (end 150.74 129.26) (width 0.2) (layer "F.Cu") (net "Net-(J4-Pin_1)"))
 (segment (start 110.96 126.96) (end 108 124) (width 0.2) (layer "F.Cu") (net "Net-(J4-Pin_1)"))
 (segment (start 108 114) (end 108.05 113.95) (width 0.2) (layer "F.Cu") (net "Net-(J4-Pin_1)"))
 (segment (start 115.055 113.95) (end 121.465 107.54) (width 0.2) (layer "F.Cu") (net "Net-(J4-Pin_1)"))
 (segment (start 110.96 132.08) (end 110.96 126.96) (width 0.2) (layer "F.Cu") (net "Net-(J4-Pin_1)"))
 (segment (start 113.875 113.95) (end 115.055 113.95) (width 0.2) (layer "F.Cu") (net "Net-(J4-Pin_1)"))
 (segment (start 153 107.54) (end 153 114.925) (width 0.2) (layer "F.Cu") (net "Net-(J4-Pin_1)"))
 (segment (start 153 114.925) (end 156.125 118.05) (width 0.2) (layer "F.Cu") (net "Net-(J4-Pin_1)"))
 (segment (start 108 124) (end 108 114) (width 0.2) (layer "F.Cu") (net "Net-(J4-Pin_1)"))
 (segment (start 122.3 91.16) (end 133.6 102.46) (width 0.2) (layer "F.Cu") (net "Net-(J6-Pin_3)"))
 (segment (start 133.6 102.46) (end 153 102.46) (width 0.2) (layer "F.Cu") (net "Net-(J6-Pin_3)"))
 (segment (start 110.75 77.025) (end 110.75 84.975) (width 0.2) (layer "F.Cu") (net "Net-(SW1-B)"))
 (segment (start 156.46 83.54) (end 158.81 81.19) (width 0.2) (layer "B.Cu") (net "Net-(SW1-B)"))
 (segment (start 147.7 83.54) (end 156.46 83.54) (width 0.2) (layer "B.Cu") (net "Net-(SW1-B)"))
 (segment (start 147.7 83.54) (end 146.24 85) (width 0.2) (layer "B.Cu") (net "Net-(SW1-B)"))
 (segment (start 146.24 85) (end 114 85) (width 0.2) (layer "B.Cu") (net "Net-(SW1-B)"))
 (segment (start 114 85) (end 112 85) (width 0.2) (layer "B.Cu") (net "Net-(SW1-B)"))
 (segment (start 158.81 81.19) (end 158.81 76) (width 0.2) (layer "B.Cu") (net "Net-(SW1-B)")))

